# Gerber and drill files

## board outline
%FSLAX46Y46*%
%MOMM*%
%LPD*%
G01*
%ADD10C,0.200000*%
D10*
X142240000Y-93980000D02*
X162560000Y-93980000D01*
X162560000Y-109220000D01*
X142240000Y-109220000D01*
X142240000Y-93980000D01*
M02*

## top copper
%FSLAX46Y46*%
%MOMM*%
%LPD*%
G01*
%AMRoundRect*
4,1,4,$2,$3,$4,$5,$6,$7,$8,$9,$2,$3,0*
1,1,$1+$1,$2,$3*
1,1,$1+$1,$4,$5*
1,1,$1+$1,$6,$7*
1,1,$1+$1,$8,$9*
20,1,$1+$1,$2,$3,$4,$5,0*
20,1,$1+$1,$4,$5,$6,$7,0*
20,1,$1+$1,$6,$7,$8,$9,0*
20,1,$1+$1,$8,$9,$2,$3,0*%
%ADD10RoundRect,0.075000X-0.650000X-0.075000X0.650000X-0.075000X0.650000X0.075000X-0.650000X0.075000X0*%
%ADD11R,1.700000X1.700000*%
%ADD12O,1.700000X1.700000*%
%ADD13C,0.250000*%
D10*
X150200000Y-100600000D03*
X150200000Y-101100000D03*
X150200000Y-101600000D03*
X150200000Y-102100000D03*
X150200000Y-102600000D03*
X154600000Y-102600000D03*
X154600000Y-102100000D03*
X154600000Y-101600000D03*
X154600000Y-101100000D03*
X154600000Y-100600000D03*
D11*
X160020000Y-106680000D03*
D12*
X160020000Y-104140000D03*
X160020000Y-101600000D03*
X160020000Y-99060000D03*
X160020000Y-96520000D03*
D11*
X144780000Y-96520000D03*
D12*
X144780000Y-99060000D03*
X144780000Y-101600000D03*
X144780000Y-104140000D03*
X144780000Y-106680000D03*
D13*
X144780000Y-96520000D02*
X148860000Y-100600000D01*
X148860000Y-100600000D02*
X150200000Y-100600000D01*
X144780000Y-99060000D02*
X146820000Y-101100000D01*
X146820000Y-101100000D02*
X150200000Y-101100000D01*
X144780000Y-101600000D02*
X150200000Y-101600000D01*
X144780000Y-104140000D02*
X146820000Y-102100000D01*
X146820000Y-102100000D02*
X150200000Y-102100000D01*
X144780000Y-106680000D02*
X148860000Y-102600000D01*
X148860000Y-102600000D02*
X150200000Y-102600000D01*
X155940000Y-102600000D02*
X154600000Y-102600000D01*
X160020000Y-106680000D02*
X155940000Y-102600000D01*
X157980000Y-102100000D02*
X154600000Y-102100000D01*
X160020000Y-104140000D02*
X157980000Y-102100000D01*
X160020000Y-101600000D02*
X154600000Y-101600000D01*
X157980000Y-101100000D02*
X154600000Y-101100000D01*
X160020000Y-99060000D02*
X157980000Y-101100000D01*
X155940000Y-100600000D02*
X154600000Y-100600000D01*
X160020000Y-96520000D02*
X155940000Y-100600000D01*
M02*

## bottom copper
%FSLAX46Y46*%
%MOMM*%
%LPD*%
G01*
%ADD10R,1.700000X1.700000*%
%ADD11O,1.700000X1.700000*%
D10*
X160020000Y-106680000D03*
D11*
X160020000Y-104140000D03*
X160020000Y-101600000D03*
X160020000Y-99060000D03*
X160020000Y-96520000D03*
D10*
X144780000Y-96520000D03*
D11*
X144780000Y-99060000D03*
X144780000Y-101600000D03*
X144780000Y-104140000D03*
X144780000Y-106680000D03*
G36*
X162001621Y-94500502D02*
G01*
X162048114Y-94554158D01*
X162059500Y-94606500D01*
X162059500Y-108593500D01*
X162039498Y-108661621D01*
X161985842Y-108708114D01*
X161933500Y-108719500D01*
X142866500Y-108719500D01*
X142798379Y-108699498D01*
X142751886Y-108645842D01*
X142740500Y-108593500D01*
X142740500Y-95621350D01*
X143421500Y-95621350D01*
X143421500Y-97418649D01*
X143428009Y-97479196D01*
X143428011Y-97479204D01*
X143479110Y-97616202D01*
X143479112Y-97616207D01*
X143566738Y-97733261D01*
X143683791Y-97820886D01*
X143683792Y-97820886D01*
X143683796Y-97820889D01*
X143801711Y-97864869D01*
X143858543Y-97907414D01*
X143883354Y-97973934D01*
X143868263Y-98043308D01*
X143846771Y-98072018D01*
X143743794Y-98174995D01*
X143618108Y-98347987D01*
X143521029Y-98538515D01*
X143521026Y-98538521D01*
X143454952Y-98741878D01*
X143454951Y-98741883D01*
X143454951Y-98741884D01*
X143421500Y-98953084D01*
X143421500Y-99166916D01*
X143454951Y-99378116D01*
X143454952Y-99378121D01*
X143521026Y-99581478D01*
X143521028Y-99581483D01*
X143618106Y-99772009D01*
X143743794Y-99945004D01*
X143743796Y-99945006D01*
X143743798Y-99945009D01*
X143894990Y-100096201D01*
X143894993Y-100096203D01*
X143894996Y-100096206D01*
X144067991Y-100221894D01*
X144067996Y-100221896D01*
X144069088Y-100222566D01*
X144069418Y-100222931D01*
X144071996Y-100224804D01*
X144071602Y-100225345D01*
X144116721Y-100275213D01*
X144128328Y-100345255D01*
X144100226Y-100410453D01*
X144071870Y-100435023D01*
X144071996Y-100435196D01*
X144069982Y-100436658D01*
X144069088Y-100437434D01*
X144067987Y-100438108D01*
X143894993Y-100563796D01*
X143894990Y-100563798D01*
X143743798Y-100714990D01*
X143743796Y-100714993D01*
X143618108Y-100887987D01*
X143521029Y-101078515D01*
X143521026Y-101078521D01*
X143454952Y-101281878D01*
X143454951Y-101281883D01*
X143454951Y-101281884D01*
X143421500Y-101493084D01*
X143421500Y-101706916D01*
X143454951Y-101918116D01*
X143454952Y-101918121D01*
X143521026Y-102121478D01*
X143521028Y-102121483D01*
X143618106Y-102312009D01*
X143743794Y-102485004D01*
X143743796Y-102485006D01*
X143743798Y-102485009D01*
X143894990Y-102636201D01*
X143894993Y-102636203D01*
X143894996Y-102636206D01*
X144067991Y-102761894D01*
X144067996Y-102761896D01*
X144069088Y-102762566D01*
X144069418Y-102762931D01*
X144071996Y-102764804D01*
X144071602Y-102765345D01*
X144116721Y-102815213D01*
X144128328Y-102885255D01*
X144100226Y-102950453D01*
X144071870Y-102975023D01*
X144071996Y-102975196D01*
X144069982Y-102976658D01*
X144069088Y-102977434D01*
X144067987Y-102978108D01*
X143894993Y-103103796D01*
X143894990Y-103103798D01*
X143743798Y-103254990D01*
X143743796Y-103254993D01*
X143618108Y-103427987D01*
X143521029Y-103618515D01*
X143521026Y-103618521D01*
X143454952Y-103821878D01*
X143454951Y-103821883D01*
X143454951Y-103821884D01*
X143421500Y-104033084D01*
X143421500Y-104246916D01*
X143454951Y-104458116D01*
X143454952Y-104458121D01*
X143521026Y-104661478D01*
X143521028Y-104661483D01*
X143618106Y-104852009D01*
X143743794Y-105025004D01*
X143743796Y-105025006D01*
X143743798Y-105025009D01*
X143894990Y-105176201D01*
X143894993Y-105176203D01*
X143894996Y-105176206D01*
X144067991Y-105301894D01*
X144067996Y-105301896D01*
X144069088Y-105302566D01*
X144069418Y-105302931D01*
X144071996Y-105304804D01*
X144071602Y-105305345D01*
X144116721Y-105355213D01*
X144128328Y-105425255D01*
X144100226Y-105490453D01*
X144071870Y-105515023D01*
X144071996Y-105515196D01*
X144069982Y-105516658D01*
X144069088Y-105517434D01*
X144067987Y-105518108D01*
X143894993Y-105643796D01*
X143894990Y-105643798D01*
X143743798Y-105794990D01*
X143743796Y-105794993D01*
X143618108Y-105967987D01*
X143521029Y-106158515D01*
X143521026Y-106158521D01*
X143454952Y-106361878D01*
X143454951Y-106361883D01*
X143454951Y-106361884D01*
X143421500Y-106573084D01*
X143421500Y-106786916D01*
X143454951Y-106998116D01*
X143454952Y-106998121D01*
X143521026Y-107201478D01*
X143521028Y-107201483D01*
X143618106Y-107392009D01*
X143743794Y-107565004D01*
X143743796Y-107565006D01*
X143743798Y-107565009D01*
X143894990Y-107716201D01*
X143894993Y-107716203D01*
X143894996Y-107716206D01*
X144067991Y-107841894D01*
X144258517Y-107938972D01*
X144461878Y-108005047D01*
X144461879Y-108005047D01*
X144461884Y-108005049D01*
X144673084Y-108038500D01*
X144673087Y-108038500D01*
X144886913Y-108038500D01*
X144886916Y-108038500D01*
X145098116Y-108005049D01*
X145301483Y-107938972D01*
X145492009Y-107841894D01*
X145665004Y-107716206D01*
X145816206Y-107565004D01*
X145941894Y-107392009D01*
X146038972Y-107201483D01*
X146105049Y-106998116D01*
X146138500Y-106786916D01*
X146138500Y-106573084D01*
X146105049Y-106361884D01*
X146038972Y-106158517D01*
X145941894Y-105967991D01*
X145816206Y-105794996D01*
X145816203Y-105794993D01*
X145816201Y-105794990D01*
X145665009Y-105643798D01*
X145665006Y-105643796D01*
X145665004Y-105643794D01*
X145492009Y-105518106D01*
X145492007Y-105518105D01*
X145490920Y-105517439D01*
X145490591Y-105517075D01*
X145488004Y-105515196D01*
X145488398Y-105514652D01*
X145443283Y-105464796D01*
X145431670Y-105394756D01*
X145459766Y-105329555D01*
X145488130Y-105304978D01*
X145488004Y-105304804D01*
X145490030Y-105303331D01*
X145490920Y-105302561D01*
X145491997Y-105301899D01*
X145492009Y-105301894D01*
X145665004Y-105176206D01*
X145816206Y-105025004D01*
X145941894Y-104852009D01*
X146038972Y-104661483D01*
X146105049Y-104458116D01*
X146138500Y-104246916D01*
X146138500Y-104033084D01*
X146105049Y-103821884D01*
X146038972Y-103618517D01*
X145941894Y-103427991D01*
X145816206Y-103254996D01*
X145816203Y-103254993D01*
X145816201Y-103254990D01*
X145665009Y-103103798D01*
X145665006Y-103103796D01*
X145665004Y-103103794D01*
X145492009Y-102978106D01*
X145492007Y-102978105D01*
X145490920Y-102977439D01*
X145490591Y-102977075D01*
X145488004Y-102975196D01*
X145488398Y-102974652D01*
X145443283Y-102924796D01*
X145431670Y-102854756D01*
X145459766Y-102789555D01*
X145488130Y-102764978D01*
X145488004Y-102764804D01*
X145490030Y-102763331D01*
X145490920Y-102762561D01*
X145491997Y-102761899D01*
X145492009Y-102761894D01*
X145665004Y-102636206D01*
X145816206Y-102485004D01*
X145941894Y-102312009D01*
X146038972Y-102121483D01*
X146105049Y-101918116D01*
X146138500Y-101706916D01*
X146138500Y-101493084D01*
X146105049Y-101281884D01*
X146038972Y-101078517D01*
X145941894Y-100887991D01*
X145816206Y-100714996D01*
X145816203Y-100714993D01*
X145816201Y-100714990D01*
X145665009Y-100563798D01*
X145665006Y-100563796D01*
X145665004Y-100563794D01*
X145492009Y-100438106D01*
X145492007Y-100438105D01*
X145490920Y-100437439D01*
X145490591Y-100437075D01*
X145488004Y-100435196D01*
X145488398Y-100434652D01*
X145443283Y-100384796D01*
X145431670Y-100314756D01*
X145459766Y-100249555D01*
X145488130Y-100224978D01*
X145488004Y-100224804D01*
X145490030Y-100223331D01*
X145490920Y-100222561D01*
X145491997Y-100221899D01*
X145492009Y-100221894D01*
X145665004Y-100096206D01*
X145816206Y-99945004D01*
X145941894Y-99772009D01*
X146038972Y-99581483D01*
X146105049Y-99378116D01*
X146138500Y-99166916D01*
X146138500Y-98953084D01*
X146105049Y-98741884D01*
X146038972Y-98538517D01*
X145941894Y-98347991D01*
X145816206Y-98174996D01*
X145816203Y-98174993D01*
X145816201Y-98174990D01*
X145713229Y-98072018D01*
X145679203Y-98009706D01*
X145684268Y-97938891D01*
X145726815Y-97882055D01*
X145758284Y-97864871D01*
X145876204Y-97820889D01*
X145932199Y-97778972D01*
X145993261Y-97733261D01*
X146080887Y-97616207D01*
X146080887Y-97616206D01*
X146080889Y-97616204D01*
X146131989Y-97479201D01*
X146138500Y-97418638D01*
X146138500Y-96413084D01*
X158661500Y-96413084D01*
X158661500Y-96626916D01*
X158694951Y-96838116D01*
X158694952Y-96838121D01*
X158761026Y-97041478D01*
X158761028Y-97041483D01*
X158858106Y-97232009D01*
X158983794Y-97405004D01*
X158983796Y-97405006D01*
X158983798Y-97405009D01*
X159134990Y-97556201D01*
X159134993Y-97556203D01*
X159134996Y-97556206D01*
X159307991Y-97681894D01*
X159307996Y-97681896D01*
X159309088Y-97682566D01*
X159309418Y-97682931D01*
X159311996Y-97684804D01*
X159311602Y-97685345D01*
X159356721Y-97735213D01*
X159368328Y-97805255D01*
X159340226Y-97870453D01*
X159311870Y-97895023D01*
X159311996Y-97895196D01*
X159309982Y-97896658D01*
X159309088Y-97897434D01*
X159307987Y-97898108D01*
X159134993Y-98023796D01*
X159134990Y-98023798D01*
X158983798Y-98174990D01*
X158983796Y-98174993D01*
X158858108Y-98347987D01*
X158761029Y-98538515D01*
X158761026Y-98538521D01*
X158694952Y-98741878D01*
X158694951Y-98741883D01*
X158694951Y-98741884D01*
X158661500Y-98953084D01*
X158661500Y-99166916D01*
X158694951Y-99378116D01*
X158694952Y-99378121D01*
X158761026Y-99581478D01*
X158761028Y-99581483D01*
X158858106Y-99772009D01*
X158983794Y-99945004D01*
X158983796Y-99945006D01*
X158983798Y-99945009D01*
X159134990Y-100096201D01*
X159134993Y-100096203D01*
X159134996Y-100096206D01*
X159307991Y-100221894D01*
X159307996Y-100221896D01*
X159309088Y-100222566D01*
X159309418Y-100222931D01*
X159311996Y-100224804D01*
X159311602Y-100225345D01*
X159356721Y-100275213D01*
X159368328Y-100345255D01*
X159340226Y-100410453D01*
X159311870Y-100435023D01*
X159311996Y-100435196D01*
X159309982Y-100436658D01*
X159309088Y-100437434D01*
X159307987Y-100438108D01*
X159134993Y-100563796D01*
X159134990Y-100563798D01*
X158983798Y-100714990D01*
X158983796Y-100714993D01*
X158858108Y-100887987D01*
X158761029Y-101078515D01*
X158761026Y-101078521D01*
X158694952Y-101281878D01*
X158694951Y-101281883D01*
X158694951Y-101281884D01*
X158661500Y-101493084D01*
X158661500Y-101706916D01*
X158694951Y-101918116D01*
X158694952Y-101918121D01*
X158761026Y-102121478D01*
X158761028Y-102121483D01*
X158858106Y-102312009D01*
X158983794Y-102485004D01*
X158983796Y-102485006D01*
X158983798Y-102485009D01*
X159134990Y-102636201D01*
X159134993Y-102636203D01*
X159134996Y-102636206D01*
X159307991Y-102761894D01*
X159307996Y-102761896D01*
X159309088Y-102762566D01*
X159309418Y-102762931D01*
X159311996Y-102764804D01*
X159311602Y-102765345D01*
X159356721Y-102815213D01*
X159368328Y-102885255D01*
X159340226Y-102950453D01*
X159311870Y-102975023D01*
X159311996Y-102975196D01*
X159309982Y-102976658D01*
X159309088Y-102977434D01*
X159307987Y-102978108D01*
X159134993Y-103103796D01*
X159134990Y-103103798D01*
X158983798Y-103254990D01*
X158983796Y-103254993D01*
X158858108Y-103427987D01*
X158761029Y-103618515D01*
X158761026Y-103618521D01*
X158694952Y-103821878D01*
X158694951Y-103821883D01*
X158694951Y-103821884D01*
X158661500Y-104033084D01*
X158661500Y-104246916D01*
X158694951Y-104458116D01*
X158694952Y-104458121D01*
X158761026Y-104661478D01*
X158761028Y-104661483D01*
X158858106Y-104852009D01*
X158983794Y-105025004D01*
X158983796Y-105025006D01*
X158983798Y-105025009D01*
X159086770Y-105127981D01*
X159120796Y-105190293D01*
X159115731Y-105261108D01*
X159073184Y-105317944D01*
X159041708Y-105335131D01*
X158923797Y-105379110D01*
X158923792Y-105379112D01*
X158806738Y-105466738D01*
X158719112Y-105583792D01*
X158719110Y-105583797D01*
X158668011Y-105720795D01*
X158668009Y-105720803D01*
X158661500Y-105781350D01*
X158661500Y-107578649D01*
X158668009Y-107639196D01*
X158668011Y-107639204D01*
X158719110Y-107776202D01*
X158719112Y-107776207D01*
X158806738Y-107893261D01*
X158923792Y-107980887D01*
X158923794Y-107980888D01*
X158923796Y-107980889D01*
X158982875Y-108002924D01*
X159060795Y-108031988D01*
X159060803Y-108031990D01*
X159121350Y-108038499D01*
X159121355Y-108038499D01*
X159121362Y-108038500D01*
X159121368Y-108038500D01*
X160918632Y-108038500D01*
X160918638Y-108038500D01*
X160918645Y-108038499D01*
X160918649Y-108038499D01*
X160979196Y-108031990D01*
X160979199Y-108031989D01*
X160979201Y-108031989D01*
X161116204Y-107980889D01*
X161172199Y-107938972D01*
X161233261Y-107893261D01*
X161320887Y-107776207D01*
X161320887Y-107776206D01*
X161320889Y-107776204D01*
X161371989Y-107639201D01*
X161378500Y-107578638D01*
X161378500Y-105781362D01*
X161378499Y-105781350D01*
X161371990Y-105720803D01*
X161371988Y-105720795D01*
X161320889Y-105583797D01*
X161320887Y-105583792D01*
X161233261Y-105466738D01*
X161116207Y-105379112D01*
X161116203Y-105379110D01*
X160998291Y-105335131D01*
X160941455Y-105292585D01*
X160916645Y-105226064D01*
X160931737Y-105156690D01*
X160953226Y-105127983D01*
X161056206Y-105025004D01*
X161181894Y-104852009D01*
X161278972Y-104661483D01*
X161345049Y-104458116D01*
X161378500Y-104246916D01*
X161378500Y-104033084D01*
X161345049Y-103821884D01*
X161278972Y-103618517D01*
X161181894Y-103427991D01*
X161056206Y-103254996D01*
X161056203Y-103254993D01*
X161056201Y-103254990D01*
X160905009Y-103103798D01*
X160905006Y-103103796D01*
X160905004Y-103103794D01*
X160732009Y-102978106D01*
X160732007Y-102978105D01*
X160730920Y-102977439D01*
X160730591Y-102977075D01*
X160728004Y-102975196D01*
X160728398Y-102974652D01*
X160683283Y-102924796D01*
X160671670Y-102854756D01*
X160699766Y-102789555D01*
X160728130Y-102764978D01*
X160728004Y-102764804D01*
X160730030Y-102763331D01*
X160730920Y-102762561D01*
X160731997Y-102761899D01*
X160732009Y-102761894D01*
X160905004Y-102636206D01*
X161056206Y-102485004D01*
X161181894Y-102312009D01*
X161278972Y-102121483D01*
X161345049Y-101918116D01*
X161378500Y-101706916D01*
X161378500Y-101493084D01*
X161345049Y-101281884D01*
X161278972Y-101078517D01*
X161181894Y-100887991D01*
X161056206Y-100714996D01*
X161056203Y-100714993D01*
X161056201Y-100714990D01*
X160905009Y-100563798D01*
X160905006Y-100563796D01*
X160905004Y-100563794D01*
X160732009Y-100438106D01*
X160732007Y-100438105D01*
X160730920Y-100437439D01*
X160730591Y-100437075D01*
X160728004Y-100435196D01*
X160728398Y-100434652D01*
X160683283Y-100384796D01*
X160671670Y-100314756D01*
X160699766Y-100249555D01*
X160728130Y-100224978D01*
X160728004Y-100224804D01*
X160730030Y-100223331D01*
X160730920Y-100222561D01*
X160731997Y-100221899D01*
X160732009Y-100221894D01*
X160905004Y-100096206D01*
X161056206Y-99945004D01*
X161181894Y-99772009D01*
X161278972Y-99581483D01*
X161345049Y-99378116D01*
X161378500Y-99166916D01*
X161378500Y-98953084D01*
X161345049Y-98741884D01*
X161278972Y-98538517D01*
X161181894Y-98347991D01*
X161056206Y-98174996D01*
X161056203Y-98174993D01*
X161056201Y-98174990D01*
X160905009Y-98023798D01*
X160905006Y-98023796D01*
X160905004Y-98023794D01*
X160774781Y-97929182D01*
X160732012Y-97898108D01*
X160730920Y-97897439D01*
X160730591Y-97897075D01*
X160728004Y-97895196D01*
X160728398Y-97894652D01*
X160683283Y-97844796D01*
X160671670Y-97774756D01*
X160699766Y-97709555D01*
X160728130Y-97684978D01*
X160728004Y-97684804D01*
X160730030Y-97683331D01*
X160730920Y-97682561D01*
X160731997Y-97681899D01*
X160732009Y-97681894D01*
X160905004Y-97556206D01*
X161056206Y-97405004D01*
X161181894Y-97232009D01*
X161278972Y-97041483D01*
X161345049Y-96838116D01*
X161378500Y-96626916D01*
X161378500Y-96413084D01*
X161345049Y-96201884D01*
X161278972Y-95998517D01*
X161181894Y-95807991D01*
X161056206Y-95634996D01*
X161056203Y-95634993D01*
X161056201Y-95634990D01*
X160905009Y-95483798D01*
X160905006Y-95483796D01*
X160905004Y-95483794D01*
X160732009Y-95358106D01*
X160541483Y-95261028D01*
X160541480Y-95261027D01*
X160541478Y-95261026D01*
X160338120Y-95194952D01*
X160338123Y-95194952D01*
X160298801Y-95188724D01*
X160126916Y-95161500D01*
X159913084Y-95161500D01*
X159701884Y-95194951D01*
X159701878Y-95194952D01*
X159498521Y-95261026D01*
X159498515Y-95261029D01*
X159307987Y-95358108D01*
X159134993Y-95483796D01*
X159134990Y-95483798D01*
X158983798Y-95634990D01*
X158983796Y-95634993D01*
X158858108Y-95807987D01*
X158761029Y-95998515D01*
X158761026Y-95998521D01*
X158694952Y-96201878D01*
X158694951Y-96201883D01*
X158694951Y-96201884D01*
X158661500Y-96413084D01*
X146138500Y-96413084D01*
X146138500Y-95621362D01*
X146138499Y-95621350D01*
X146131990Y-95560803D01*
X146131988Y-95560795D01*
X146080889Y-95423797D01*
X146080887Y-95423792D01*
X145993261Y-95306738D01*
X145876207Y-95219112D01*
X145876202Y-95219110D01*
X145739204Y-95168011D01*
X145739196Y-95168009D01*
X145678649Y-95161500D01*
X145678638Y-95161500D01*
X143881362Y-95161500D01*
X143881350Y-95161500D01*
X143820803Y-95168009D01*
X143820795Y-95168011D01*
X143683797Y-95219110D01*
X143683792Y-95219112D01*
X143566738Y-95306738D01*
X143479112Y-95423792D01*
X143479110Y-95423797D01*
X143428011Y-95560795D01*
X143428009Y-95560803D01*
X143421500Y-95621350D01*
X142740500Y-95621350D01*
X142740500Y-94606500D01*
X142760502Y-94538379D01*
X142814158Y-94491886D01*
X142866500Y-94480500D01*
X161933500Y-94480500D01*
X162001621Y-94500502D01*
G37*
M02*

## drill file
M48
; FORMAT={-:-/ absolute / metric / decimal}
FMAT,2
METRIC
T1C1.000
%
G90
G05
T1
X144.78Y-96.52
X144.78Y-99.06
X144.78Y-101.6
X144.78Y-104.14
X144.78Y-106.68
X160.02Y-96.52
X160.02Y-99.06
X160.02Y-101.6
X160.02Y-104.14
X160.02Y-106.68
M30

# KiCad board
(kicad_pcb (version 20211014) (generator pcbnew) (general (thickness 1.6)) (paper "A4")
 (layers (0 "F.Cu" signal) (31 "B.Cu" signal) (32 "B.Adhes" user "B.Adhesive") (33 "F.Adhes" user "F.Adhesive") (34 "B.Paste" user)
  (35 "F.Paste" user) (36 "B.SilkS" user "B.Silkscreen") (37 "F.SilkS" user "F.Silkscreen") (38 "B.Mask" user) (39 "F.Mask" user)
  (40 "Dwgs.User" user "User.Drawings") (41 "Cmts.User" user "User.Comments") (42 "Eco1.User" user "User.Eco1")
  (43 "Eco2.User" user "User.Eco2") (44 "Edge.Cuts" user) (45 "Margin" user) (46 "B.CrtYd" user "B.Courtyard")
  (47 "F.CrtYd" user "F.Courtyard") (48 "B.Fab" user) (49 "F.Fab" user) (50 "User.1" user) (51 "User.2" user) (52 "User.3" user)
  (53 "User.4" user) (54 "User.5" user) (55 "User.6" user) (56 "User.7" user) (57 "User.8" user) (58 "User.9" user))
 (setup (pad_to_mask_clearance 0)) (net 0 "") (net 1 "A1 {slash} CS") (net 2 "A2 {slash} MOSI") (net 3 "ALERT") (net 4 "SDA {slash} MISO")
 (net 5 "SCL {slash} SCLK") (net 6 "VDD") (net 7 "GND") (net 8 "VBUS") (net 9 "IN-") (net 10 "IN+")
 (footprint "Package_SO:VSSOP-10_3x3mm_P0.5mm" (layer "F.Cu") (at 152.4 101.6)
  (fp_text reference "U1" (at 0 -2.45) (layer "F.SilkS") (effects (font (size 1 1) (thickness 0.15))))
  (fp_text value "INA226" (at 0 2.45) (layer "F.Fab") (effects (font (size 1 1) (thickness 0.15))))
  (pad "1" smd roundrect (at -2.2 -1) (size 1.45 0.3) (layers "F.Cu" "F.Paste" "F.Mask") (roundrect_rratio 0.25) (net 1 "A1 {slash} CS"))
  (pad "2" smd roundrect (at -2.2 -0.5) (size 1.45 0.3) (layers "F.Cu" "F.Paste" "F.Mask") (roundrect_rratio 0.25) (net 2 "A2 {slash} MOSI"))
  (pad "3" smd roundrect (at -2.2 0) (size 1.45 0.3) (layers "F.Cu" "F.Paste" "F.Mask") (roundrect_rratio 0.25) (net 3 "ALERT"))
  (pad "4" smd roundrect (at -2.2 0.5) (size 1.45 0.3) (layers "F.Cu" "F.Paste" "F.Mask") (roundrect_rratio 0.25) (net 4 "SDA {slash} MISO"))
  (pad "5" smd roundrect (at -2.2 1) (size 1.45 0.3) (layers "F.Cu" "F.Paste" "F.Mask") (roundrect_rratio 0.25) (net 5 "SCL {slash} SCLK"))
  (pad "6" smd roundrect (at 2.2 1) (size 1.45 0.3) (layers "F.Cu" "F.Paste" "F.Mask") (roundrect_rratio 0.25) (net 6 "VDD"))
  (pad "7" smd roundrect (at 2.2 0.5) (size 1.45 0.3) (layers "F.Cu" "F.Paste" "F.Mask") (roundrect_rratio 0.25) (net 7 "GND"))
  (pad "8" smd roundrect (at 2.2 0) (size 1.45 0.3) (layers "F.Cu" "F.Paste" "F.Mask") (roundrect_rratio 0.25) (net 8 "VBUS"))
  (pad "9" smd roundrect (at 2.2 -0.5) (size 1.45 0.3) (layers "F.Cu" "F.Paste" "F.Mask") (roundrect_rratio 0.25) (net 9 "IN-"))
  (pad "10" smd roundrect (at 2.2 -1) (size 1.45 0.3) (layers "F.Cu" "F.Paste" "F.Mask") (roundrect_rratio 0.25) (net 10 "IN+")))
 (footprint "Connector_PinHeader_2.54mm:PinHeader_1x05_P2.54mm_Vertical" (layer "B.Cu") (at 160.02 106.68)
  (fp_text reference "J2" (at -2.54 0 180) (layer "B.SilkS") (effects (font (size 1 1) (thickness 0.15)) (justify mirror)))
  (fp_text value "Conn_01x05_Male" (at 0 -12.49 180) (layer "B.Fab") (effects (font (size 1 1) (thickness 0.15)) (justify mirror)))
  (pad "1" thru_hole rect (at 0 0) (size 1.7 1.7) (drill 1) (layers *.Cu *.Mask) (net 6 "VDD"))
  (pad "2" thru_hole oval (at 0 -2.54) (size 1.7 1.7) (drill 1) (layers *.Cu *.Mask) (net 7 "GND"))
  (pad "3" thru_hole oval (at 0 -5.08) (size 1.7 1.7) (drill 1) (layers *.Cu *.Mask) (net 8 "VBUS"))
  (pad "4" thru_hole oval (at 0 -7.62) (size 1.7 1.7) (drill 1) (layers *.Cu *.Mask) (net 9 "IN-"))
  (pad "5" thru_hole oval (at 0 -10.16) (size 1.7 1.7) (drill 1) (layers *.Cu *.Mask) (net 10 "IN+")))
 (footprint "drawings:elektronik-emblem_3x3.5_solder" (layer "B.Cu") (at 152.4 97.155 180)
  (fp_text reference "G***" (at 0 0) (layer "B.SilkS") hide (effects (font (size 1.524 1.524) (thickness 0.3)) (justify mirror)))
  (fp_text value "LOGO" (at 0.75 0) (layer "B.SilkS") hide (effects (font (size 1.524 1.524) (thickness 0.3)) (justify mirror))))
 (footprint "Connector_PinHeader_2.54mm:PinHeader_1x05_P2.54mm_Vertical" (layer "B.Cu") (at 144.78 96.52 180)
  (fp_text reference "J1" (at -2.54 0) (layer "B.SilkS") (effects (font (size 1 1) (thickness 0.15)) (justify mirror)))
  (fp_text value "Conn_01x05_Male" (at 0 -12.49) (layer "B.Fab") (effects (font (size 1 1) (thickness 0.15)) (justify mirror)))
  (pad "1" thru_hole rect (at 0 0 180) (size 1.7 1.7) (drill 1) (layers *.Cu *.Mask) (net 1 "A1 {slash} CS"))
  (pad "2" thru_hole oval (at 0 -2.54 180) (size 1.7 1.7) (drill 1) (layers *.Cu *.Mask) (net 2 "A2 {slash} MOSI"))
  (pad "3" thru_hole oval (at 0 -5.08 180) (size 1.7 1.7) (drill 1) (layers *.Cu *.Mask) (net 3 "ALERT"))
  (pad "4" thru_hole oval (at 0 -7.62 180) (size 1.7 1.7) (drill 1) (layers *.Cu *.Mask) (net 4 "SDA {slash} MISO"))
  (pad "5" thru_hole oval (at 0 -10.16 180) (size 1.7 1.7) (drill 1) (layers *.Cu *.Mask) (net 5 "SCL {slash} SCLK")))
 (gr_rect (start 142.24 93.98) (end 162.56 109.22) (layer "Edge.Cuts") (width 0.2) (fill none))
 (segment (start 144.78 96.52) (end 148.86 100.6) (width 0.25) (layer "F.Cu") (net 1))
 (segment (start 148.86 100.6) (end 150.2 100.6) (width 0.25) (layer "F.Cu") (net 1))
 (segment (start 144.78 99.06) (end 146.82 101.1) (width 0.25) (layer "F.Cu") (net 2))
 (segment (start 146.82 101.1) (end 150.2 101.1) (width 0.25) (layer "F.Cu") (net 2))
 (segment (start 144.78 101.6) (end 150.2 101.6) (width 0.25) (layer "F.Cu") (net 3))
 (segment (start 144.78 104.14) (end 146.82 102.1) (width 0.25) (layer "F.Cu") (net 4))
 (segment (start 146.82 102.1) (end 150.2 102.1) (width 0.25) (layer "F.Cu") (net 4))
 (segment (start 144.78 106.68) (end 148.86 102.6) (width 0.25) (layer "F.Cu") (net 5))
 (segment (start 148.86 102.6) (end 150.2 102.6) (width 0.25) (layer "F.Cu") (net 5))
 (segment (start 155.94 102.6) (end 154.6 102.6) (width 0.25) (layer "F.Cu") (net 6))
 (segment (start 160.02 106.68) (end 155.94 102.6) (width 0.25) (layer "F.Cu") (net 6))
 (segment (start 157.98 102.1) (end 154.6 102.1) (width 0.25) (layer "F.Cu") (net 7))
 (segment (start 160.02 104.14) (end 157.98 102.1) (width 0.25) (layer "F.Cu") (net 7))
 (segment (start 160.02 101.6) (end 154.6 101.6) (width 0.25) (layer "F.Cu") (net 8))
 (segment (start 157.98 101.1) (end 154.6 101.1) (width 0.25) (layer "F.Cu") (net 9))
 (segment (start 160.02 99.06) (end 157.98 101.1) (width 0.25) (layer "F.Cu") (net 9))
 (segment (start 155.94 100.6) (end 154.6 100.6) (width 0.25) (layer "F.Cu") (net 10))
 (segment (start 160.02 96.52) (end 155.94 100.6) (width 0.25) (layer "F.Cu") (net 10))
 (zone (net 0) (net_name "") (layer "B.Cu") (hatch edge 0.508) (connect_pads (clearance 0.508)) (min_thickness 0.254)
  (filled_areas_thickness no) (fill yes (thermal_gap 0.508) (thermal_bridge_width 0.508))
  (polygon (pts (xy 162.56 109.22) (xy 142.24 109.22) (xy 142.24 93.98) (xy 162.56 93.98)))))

